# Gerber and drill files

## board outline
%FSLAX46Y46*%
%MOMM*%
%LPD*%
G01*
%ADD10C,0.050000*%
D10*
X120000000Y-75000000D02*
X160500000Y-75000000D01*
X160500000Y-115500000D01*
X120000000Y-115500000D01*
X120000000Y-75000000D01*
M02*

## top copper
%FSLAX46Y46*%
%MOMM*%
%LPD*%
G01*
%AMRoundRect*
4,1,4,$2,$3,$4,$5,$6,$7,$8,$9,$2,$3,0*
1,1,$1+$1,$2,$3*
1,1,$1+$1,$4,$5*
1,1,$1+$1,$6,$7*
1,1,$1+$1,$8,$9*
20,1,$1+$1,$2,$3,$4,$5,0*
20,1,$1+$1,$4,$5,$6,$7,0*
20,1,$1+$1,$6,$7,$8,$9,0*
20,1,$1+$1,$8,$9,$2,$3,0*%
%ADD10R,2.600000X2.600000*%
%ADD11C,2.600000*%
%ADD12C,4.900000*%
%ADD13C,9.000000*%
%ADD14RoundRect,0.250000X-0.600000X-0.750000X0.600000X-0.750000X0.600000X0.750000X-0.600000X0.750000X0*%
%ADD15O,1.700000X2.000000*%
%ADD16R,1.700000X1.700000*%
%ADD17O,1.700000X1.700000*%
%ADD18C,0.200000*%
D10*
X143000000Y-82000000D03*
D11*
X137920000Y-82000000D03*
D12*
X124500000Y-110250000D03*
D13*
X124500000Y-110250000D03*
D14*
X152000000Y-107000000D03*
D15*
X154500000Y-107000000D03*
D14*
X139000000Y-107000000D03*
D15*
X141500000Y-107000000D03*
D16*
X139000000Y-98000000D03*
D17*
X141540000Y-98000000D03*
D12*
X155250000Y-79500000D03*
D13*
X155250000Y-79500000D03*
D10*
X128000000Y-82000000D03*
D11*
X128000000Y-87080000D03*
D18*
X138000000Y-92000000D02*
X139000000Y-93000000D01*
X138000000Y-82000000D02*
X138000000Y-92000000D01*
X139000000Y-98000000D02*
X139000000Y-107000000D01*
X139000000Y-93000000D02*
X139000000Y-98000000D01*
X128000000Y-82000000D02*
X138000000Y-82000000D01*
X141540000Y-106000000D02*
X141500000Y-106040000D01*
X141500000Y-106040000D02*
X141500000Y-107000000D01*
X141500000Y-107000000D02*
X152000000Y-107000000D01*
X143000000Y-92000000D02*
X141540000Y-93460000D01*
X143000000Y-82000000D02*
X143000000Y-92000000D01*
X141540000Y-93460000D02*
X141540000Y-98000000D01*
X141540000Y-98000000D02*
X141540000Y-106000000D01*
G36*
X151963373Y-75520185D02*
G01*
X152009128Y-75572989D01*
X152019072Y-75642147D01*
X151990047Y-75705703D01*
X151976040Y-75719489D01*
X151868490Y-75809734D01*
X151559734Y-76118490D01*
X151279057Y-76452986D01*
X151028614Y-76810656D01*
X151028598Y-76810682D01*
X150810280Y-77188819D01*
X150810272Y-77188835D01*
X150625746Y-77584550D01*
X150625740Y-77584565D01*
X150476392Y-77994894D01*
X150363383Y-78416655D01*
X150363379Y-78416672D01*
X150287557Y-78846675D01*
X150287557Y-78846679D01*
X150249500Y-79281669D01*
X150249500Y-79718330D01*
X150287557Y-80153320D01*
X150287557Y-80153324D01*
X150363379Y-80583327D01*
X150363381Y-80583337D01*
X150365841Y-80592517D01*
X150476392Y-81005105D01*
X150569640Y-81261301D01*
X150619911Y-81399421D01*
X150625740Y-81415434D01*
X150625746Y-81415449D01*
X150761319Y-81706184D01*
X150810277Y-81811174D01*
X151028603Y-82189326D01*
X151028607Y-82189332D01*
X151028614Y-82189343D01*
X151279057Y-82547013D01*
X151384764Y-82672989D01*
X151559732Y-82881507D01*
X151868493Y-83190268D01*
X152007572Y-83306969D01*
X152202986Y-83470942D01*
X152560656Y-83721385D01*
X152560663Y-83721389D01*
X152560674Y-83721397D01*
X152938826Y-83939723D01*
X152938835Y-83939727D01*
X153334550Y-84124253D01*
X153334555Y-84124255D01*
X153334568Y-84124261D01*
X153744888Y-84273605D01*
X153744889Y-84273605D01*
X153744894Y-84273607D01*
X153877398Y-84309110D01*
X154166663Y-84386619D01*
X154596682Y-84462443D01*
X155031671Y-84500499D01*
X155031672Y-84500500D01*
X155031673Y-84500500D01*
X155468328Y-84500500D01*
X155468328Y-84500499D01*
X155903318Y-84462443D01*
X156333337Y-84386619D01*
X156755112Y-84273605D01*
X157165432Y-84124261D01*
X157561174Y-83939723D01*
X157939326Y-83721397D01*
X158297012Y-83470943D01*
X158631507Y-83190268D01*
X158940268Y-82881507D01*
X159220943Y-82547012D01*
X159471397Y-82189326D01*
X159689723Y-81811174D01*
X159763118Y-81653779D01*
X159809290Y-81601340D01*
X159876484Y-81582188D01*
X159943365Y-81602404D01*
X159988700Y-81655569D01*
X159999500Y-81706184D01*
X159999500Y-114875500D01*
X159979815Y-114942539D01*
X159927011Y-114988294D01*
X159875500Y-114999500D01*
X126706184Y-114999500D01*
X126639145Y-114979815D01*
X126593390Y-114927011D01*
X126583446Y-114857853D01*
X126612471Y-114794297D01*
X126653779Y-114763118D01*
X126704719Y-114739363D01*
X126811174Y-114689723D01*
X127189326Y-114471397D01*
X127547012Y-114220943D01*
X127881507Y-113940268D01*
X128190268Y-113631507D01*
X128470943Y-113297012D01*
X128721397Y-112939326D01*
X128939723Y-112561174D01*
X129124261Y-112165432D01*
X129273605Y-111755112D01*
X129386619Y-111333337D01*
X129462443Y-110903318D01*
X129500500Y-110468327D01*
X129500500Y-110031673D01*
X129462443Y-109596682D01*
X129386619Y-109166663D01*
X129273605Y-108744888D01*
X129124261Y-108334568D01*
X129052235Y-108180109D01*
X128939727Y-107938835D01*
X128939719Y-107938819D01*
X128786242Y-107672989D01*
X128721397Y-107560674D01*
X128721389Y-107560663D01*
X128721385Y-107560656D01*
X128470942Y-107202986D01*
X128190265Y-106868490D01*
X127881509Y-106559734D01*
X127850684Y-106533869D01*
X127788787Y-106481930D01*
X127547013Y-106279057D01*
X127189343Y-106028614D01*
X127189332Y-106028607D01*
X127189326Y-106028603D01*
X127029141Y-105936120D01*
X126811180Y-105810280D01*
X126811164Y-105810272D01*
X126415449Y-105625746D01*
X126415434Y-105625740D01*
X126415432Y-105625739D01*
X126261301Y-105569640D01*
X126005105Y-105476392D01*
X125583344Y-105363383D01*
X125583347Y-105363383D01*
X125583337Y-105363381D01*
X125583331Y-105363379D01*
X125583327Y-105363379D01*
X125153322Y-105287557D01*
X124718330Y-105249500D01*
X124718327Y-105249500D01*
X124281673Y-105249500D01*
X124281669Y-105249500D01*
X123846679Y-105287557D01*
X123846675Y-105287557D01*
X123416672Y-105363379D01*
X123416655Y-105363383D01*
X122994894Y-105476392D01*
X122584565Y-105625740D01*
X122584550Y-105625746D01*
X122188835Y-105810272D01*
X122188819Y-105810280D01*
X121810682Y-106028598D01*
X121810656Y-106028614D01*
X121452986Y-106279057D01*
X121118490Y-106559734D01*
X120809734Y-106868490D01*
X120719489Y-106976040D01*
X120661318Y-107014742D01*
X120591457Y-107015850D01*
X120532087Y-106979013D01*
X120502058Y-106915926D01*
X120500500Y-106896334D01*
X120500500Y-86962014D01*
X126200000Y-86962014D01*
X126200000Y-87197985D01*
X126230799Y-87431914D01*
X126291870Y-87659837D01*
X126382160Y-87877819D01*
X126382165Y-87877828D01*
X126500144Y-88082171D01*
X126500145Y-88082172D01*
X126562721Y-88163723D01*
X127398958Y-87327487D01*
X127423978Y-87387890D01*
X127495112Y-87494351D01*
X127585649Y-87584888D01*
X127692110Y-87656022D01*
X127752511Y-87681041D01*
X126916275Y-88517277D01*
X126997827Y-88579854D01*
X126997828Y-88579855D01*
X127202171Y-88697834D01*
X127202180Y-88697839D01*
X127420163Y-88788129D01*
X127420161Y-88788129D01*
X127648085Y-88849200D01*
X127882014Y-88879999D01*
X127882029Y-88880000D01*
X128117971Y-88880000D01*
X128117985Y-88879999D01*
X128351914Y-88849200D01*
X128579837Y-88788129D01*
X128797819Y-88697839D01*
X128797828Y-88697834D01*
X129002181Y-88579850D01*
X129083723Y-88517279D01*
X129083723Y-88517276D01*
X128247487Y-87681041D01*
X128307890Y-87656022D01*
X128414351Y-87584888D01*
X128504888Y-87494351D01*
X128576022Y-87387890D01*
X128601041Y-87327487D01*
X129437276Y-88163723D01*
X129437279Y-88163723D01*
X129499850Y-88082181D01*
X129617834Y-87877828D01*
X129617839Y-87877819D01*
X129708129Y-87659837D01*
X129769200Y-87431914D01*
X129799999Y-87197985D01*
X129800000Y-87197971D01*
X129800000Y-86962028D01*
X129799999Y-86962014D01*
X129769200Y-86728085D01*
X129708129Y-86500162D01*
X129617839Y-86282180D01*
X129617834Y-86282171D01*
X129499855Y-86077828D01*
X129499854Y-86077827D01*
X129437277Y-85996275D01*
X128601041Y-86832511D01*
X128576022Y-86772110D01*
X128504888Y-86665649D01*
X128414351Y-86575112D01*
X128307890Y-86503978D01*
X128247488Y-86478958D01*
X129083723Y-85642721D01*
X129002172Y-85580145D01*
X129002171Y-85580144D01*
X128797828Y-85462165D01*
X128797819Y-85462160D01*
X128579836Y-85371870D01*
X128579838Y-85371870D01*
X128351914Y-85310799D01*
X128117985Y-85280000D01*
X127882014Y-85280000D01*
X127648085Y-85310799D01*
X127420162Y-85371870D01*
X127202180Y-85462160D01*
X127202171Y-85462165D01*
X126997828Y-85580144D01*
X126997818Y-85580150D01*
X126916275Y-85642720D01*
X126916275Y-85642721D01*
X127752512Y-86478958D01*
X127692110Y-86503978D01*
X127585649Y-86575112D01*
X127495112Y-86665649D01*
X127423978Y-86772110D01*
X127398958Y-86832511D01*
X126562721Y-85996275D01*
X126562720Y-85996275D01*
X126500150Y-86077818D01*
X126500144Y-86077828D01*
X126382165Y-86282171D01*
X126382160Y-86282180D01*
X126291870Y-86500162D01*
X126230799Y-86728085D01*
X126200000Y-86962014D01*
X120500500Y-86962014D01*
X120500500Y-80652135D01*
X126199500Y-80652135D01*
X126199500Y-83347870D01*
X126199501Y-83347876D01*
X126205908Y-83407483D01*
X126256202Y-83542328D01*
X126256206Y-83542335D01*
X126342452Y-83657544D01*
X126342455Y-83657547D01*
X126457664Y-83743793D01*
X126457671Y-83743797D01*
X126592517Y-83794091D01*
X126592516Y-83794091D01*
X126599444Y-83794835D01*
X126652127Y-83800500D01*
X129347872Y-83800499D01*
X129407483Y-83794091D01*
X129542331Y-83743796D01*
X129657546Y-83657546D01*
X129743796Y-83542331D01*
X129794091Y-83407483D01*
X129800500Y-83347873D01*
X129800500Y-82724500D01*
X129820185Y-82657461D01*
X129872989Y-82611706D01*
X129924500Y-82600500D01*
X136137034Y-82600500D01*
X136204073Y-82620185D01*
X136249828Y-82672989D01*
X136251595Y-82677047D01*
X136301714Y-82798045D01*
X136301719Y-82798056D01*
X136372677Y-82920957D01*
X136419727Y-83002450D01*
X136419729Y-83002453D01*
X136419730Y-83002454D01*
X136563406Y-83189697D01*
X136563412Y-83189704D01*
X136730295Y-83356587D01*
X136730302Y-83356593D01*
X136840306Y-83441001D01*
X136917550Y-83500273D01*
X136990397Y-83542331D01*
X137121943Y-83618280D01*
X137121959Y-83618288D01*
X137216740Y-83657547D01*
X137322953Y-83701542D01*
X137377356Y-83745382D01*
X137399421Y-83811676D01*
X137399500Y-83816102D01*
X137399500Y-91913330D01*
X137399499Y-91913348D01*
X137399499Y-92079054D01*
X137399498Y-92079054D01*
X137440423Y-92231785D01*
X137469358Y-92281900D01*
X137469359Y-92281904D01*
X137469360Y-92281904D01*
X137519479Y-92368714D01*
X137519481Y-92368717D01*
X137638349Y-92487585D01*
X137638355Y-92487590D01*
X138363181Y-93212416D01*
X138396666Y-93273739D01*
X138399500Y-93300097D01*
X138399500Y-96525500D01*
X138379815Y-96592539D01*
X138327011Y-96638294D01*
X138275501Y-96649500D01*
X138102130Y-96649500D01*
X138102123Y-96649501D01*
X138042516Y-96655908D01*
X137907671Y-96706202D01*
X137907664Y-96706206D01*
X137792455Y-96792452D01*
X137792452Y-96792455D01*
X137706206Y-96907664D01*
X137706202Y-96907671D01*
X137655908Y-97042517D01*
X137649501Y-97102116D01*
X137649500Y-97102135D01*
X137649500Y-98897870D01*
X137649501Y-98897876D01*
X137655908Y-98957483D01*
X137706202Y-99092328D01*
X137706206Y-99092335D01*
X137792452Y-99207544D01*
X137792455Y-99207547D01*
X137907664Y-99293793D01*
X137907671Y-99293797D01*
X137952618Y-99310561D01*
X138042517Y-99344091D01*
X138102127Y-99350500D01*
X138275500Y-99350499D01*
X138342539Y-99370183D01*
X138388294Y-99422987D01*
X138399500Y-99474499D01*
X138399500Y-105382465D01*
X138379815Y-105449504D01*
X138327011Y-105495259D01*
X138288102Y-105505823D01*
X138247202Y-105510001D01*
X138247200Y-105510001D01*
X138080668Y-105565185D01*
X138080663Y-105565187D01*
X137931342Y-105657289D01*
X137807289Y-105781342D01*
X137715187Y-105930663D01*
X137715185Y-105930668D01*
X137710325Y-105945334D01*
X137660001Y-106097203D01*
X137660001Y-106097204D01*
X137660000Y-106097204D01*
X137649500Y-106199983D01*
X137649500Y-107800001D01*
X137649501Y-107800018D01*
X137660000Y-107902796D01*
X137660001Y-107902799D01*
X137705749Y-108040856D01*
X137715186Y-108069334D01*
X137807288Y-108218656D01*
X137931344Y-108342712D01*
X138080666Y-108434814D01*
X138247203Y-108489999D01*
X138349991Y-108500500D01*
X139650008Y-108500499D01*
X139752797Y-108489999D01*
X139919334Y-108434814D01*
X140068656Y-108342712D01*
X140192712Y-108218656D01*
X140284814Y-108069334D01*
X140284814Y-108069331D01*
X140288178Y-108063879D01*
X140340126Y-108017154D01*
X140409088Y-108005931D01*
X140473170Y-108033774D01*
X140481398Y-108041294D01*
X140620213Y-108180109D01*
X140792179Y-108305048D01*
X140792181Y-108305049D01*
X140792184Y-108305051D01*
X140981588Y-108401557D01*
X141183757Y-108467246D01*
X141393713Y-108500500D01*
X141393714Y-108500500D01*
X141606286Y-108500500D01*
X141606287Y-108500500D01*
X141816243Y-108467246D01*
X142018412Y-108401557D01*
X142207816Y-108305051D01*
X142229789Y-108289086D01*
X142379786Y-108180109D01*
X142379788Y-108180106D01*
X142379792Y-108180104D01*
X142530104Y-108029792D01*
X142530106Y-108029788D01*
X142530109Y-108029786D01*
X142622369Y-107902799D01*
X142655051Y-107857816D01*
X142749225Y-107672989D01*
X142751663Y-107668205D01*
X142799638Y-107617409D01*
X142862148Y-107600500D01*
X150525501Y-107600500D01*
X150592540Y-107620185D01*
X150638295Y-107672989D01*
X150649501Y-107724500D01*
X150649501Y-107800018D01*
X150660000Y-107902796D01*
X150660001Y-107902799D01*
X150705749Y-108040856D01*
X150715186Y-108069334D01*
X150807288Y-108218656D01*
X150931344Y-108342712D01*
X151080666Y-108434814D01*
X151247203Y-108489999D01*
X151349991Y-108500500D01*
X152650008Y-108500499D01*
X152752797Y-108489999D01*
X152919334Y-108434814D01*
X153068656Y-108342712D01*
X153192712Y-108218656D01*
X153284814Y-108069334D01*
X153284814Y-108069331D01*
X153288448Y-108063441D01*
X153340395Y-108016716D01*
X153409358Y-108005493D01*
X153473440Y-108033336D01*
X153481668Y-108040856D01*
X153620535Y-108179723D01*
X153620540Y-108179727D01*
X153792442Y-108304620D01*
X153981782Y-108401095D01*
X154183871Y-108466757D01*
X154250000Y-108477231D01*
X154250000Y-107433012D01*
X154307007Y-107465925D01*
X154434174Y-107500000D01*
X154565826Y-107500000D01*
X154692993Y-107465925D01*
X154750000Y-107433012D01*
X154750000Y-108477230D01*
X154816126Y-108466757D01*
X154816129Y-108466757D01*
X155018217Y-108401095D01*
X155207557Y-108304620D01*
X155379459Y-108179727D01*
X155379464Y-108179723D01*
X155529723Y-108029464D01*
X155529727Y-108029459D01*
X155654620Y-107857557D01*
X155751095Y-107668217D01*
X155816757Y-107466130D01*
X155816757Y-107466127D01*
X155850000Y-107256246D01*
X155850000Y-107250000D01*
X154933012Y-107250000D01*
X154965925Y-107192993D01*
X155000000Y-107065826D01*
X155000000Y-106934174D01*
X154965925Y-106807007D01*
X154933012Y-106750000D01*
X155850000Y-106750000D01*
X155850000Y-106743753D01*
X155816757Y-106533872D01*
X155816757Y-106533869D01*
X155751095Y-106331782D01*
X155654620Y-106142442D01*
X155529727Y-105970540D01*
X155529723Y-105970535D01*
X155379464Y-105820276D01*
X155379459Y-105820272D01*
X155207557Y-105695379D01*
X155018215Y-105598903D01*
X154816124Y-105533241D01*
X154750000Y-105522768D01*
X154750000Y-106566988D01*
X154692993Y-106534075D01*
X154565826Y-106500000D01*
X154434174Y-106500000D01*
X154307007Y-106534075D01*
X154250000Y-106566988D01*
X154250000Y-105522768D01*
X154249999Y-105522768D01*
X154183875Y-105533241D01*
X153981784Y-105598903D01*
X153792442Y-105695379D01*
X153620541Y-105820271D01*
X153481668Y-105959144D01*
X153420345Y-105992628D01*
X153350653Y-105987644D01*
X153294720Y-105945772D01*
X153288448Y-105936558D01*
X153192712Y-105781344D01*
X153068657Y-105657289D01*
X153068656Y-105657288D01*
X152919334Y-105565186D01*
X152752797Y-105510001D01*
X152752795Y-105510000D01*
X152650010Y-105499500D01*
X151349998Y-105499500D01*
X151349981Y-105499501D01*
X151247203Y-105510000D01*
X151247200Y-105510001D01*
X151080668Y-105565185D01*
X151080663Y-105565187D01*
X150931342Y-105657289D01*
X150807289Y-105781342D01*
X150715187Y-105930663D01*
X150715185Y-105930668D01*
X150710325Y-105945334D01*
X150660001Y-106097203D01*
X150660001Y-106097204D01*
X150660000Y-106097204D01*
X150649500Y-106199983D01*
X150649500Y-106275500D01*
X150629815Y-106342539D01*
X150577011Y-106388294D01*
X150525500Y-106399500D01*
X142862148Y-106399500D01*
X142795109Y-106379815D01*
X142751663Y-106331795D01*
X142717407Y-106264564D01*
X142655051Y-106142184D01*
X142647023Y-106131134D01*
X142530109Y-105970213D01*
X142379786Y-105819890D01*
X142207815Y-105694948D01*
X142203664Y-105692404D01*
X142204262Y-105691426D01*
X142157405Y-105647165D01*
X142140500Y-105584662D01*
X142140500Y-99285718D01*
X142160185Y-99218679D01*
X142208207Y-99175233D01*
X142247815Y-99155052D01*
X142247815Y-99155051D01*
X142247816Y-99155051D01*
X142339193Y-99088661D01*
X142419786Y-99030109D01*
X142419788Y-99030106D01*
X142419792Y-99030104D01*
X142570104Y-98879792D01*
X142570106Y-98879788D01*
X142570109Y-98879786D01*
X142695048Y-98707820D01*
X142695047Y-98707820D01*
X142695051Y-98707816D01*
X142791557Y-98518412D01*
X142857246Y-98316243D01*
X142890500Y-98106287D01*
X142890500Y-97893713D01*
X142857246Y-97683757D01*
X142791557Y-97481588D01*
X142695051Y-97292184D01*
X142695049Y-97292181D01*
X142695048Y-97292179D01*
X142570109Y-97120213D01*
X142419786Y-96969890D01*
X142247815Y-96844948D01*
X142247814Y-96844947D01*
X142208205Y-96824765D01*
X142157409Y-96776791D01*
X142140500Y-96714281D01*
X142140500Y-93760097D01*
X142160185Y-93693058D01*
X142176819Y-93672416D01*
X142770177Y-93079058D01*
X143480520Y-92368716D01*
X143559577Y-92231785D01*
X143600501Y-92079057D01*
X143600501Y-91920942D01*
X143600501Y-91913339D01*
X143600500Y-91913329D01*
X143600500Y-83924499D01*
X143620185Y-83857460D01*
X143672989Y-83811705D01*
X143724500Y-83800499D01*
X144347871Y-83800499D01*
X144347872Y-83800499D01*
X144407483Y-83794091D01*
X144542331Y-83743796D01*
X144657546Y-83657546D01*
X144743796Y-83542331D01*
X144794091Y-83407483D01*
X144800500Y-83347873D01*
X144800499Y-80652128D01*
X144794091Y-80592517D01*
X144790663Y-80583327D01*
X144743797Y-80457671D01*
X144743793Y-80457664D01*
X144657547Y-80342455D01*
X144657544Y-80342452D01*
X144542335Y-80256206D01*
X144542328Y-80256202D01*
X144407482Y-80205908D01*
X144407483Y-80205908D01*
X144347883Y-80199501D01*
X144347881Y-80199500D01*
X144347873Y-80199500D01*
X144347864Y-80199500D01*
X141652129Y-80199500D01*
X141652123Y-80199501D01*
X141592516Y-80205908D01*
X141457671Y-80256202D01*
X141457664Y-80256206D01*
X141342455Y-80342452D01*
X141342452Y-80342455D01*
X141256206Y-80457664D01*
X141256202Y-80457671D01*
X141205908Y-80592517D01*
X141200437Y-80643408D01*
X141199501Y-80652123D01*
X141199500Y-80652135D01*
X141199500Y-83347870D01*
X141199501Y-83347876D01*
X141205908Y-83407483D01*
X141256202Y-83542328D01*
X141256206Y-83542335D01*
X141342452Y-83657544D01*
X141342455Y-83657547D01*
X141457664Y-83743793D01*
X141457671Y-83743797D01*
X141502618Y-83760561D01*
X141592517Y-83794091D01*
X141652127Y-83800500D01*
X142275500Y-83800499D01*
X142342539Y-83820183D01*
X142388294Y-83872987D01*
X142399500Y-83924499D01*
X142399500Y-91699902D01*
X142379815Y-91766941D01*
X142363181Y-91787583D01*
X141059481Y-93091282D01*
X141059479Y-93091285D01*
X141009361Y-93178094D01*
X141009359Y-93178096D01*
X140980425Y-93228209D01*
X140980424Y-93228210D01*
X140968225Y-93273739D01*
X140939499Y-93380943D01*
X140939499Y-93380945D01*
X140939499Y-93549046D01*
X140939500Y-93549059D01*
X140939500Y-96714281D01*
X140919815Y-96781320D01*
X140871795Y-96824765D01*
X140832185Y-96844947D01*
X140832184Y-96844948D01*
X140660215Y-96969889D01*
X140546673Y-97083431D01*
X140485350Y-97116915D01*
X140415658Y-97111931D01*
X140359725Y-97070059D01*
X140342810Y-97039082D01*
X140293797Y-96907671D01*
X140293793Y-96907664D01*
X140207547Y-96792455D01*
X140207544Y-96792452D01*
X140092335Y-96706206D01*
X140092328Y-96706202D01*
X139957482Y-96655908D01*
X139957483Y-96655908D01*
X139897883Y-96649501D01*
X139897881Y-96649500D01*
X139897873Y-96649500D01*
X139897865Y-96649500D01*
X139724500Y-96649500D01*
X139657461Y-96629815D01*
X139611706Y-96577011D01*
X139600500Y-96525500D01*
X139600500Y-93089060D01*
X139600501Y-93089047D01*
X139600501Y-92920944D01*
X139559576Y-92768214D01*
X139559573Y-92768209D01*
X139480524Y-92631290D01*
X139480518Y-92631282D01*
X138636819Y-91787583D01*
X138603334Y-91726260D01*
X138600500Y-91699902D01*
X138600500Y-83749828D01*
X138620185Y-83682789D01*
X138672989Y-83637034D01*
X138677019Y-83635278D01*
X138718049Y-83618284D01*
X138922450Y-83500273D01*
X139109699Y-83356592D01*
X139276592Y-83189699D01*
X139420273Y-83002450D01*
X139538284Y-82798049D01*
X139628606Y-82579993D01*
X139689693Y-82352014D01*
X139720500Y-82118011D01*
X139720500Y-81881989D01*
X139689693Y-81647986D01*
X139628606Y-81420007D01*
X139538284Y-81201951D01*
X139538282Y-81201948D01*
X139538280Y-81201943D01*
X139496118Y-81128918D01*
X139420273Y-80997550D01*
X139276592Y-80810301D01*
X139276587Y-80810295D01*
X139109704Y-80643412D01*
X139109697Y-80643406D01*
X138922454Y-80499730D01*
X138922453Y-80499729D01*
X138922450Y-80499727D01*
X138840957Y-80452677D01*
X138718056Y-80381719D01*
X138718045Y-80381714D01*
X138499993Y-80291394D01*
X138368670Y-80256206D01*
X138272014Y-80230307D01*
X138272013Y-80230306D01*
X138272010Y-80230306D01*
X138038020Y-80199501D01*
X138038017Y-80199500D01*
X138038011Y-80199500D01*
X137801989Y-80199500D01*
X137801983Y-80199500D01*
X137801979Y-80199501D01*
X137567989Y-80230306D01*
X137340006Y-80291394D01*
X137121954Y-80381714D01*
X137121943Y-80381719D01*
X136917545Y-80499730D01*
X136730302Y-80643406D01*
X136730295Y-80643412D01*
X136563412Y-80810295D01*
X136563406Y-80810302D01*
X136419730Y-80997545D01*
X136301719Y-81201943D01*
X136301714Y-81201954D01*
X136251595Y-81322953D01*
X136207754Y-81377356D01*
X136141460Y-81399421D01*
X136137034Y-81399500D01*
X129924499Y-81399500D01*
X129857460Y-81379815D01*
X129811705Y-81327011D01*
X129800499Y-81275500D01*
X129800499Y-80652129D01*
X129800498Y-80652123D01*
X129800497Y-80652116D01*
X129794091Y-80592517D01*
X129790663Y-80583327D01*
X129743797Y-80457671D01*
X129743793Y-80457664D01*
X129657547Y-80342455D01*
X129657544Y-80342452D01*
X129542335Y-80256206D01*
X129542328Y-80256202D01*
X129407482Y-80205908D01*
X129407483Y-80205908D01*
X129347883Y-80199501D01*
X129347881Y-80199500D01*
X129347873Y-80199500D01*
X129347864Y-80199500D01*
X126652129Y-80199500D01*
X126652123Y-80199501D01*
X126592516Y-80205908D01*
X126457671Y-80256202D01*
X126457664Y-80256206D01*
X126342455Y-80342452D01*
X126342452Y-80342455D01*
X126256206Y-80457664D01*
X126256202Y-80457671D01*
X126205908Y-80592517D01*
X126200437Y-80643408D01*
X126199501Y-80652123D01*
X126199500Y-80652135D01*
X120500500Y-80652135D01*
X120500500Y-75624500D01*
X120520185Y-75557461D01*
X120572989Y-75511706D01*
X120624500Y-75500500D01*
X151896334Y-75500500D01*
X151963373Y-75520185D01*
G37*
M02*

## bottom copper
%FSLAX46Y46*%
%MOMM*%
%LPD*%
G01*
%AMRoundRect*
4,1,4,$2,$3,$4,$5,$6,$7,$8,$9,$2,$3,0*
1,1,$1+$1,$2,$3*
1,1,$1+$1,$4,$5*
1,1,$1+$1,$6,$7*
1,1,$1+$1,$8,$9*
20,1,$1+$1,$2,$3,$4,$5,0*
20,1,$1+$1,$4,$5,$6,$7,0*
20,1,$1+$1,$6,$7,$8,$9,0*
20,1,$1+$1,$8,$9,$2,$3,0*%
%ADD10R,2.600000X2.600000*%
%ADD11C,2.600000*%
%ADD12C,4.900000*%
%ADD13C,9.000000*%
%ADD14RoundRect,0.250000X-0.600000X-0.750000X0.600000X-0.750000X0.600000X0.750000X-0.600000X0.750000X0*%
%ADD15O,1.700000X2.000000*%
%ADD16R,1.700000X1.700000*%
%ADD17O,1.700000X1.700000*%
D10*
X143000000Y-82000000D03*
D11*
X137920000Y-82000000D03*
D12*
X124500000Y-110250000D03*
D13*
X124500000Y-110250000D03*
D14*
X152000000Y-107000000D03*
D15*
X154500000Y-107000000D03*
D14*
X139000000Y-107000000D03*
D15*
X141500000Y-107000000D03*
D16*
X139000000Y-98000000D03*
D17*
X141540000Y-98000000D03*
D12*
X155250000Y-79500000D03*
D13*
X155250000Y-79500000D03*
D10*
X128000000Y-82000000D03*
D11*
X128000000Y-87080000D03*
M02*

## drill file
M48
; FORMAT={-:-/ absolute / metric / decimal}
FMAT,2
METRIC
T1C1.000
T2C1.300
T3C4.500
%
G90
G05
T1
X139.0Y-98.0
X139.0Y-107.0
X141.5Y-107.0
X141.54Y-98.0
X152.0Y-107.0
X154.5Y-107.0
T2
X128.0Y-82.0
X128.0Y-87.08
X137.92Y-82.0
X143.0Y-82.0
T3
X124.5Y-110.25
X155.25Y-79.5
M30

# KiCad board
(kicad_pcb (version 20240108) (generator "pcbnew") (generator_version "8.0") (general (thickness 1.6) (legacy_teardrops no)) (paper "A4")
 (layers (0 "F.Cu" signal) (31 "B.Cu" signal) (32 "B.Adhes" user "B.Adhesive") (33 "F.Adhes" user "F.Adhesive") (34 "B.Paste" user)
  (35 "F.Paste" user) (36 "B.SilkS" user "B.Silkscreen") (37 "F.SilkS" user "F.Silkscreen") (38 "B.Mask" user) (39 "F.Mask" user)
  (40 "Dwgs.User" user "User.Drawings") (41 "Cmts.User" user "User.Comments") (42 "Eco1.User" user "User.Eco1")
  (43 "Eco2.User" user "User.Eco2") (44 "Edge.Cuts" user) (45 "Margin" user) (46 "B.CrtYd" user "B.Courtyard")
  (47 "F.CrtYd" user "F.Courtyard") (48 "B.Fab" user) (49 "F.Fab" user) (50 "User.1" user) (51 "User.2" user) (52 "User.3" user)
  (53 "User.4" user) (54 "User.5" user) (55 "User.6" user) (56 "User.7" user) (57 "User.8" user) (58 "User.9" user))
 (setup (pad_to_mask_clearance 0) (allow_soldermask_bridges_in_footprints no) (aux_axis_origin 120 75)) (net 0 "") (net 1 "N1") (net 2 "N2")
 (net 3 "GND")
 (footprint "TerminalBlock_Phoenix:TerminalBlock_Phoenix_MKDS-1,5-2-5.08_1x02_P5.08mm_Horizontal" (layer "F.Cu") (at 143 82 180)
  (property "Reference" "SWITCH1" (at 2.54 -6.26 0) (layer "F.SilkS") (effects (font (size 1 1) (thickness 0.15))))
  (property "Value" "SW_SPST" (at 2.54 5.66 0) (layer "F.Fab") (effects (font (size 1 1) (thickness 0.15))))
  (pad "1" thru_hole rect (at 0 0 180) (size 2.6 2.6) (drill 1.3) (layers "*.Cu" "*.Mask") (remove_unused_layers no) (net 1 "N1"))
  (pad "2" thru_hole circle (at 5.08 0 180) (size 2.6 2.6) (drill 1.3) (layers "*.Cu" "*.Mask") (remove_unused_layers no) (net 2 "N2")))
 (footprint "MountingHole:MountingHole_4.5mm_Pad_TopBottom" (layer "F.Cu") (at 124.5 110.25)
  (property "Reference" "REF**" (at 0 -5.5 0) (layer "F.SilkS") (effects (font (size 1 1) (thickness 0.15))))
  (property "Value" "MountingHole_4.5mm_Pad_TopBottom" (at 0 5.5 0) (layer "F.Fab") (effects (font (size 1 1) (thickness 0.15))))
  (pad "1" thru_hole circle (at 0 0) (size 4.9 4.9) (drill 4.5) (layers "*.Cu" "*.Mask") (remove_unused_layers no))
  (pad "1" connect circle (at 0 0) (size 9 9) (layers "F.Cu" "F.Mask"))
  (pad "1" connect circle (at 0 0) (size 9 9) (layers "B.Cu" "B.Mask")))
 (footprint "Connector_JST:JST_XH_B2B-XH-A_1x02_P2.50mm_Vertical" (layer "F.Cu") (at 152 107)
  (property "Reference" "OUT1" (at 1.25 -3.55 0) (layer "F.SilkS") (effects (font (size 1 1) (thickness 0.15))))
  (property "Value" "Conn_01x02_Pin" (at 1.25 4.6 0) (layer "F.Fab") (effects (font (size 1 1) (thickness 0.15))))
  (pad "1" thru_hole roundrect (at 0 0) (size 1.7 2) (drill 1) (layers "*.Cu" "*.Mask") (remove_unused_layers no)
   (roundrect_rratio 0.147059) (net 1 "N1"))
  (pad "2" thru_hole oval (at 2.5 0) (size 1.7 2) (drill 1) (layers "*.Cu" "*.Mask") (remove_unused_layers no) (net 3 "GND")))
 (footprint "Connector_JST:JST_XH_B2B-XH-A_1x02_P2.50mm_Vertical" (layer "F.Cu") (at 139 107)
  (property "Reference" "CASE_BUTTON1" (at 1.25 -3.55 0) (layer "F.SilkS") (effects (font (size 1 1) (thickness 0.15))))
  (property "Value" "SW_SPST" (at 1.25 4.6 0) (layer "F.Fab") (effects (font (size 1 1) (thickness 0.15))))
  (pad "1" thru_hole roundrect (at 0 0) (size 1.7 2) (drill 1) (layers "*.Cu" "*.Mask") (remove_unused_layers no)
   (roundrect_rratio 0.147059) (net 2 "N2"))
  (pad "2" thru_hole oval (at 2.5 0) (size 1.7 2) (drill 1) (layers "*.Cu" "*.Mask") (remove_unused_layers no) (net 1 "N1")))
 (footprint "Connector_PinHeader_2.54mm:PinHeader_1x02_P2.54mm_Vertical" (layer "F.Cu") (at 139 98 90)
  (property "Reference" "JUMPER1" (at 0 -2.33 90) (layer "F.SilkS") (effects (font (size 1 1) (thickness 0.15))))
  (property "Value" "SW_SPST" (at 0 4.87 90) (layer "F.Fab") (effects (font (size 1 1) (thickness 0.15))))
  (pad "1" thru_hole rect (at 0 0 90) (size 1.7 1.7) (drill 1) (layers "*.Cu" "*.Mask") (remove_unused_layers no) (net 2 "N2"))
  (pad "2" thru_hole oval (at 0 2.54 90) (size 1.7 1.7) (drill 1) (layers "*.Cu" "*.Mask") (remove_unused_layers no) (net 1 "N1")))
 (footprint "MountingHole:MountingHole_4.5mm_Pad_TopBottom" (layer "F.Cu") (at 155.25 79.5)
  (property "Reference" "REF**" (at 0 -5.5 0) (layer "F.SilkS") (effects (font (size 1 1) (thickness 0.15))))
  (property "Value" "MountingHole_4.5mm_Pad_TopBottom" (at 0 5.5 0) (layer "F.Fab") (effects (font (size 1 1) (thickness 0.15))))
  (pad "1" thru_hole circle (at 0 0) (size 4.9 4.9) (drill 4.5) (layers "*.Cu" "*.Mask") (remove_unused_layers no))
  (pad "1" connect circle (at 0 0) (size 9 9) (layers "F.Cu" "F.Mask"))
  (pad "1" connect circle (at 0 0) (size 9 9) (layers "B.Cu" "B.Mask")))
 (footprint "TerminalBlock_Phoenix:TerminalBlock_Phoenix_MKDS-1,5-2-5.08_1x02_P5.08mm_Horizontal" (layer "F.Cu") (at 128 82 -90)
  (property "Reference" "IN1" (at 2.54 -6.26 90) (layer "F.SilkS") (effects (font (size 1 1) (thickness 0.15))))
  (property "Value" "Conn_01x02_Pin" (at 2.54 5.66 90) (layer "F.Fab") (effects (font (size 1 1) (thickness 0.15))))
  (pad "1" thru_hole rect (at 0 0 270) (size 2.6 2.6) (drill 1.3) (layers "*.Cu" "*.Mask") (remove_unused_layers no) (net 2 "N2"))
  (pad "2" thru_hole circle (at 5.08 0 270) (size 2.6 2.6) (drill 1.3) (layers "*.Cu" "*.Mask") (remove_unused_layers no) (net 3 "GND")))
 (gr_rect (start 120 75) (end 160.5 115.5) (stroke (width 0.05) (type default)) (fill none) (layer "Edge.Cuts"))
 (segment (start 138 92) (end 139 93) (width 0.2) (layer "F.Cu") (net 2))
 (segment (start 138 82) (end 138 92) (width 0.2) (layer "F.Cu") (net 2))
 (segment (start 139 98) (end 139 107) (width 0.2) (layer "F.Cu") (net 2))
 (segment (start 139 93) (end 139 98) (width 0.2) (layer "F.Cu") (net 2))
 (segment (start 128 82) (end 138 82) (width 0.2) (layer "F.Cu") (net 2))
 (segment (start 141.54 106) (end 141.5 106.04) (width 0.2) (layer "F.Cu") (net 1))
 (segment (start 141.5 106.04) (end 141.5 107) (width 0.2) (layer "F.Cu") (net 1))
 (segment (start 141.5 107) (end 152 107) (width 0.2) (layer "F.Cu") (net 1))
 (segment (start 143 92) (end 141.54 93.46) (width 0.2) (layer "F.Cu") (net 1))
 (segment (start 143 82) (end 143 92) (width 0.2) (layer "F.Cu") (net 1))
 (segment (start 141.54 93.46) (end 141.54 98) (width 0.2) (layer "F.Cu") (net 1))
 (segment (start 141.54 98) (end 141.54 106) (width 0.2) (layer "F.Cu") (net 1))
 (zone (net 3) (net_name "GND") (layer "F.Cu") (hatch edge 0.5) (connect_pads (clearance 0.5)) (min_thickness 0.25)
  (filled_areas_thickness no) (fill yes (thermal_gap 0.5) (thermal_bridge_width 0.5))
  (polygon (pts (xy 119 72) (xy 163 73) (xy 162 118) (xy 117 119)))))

